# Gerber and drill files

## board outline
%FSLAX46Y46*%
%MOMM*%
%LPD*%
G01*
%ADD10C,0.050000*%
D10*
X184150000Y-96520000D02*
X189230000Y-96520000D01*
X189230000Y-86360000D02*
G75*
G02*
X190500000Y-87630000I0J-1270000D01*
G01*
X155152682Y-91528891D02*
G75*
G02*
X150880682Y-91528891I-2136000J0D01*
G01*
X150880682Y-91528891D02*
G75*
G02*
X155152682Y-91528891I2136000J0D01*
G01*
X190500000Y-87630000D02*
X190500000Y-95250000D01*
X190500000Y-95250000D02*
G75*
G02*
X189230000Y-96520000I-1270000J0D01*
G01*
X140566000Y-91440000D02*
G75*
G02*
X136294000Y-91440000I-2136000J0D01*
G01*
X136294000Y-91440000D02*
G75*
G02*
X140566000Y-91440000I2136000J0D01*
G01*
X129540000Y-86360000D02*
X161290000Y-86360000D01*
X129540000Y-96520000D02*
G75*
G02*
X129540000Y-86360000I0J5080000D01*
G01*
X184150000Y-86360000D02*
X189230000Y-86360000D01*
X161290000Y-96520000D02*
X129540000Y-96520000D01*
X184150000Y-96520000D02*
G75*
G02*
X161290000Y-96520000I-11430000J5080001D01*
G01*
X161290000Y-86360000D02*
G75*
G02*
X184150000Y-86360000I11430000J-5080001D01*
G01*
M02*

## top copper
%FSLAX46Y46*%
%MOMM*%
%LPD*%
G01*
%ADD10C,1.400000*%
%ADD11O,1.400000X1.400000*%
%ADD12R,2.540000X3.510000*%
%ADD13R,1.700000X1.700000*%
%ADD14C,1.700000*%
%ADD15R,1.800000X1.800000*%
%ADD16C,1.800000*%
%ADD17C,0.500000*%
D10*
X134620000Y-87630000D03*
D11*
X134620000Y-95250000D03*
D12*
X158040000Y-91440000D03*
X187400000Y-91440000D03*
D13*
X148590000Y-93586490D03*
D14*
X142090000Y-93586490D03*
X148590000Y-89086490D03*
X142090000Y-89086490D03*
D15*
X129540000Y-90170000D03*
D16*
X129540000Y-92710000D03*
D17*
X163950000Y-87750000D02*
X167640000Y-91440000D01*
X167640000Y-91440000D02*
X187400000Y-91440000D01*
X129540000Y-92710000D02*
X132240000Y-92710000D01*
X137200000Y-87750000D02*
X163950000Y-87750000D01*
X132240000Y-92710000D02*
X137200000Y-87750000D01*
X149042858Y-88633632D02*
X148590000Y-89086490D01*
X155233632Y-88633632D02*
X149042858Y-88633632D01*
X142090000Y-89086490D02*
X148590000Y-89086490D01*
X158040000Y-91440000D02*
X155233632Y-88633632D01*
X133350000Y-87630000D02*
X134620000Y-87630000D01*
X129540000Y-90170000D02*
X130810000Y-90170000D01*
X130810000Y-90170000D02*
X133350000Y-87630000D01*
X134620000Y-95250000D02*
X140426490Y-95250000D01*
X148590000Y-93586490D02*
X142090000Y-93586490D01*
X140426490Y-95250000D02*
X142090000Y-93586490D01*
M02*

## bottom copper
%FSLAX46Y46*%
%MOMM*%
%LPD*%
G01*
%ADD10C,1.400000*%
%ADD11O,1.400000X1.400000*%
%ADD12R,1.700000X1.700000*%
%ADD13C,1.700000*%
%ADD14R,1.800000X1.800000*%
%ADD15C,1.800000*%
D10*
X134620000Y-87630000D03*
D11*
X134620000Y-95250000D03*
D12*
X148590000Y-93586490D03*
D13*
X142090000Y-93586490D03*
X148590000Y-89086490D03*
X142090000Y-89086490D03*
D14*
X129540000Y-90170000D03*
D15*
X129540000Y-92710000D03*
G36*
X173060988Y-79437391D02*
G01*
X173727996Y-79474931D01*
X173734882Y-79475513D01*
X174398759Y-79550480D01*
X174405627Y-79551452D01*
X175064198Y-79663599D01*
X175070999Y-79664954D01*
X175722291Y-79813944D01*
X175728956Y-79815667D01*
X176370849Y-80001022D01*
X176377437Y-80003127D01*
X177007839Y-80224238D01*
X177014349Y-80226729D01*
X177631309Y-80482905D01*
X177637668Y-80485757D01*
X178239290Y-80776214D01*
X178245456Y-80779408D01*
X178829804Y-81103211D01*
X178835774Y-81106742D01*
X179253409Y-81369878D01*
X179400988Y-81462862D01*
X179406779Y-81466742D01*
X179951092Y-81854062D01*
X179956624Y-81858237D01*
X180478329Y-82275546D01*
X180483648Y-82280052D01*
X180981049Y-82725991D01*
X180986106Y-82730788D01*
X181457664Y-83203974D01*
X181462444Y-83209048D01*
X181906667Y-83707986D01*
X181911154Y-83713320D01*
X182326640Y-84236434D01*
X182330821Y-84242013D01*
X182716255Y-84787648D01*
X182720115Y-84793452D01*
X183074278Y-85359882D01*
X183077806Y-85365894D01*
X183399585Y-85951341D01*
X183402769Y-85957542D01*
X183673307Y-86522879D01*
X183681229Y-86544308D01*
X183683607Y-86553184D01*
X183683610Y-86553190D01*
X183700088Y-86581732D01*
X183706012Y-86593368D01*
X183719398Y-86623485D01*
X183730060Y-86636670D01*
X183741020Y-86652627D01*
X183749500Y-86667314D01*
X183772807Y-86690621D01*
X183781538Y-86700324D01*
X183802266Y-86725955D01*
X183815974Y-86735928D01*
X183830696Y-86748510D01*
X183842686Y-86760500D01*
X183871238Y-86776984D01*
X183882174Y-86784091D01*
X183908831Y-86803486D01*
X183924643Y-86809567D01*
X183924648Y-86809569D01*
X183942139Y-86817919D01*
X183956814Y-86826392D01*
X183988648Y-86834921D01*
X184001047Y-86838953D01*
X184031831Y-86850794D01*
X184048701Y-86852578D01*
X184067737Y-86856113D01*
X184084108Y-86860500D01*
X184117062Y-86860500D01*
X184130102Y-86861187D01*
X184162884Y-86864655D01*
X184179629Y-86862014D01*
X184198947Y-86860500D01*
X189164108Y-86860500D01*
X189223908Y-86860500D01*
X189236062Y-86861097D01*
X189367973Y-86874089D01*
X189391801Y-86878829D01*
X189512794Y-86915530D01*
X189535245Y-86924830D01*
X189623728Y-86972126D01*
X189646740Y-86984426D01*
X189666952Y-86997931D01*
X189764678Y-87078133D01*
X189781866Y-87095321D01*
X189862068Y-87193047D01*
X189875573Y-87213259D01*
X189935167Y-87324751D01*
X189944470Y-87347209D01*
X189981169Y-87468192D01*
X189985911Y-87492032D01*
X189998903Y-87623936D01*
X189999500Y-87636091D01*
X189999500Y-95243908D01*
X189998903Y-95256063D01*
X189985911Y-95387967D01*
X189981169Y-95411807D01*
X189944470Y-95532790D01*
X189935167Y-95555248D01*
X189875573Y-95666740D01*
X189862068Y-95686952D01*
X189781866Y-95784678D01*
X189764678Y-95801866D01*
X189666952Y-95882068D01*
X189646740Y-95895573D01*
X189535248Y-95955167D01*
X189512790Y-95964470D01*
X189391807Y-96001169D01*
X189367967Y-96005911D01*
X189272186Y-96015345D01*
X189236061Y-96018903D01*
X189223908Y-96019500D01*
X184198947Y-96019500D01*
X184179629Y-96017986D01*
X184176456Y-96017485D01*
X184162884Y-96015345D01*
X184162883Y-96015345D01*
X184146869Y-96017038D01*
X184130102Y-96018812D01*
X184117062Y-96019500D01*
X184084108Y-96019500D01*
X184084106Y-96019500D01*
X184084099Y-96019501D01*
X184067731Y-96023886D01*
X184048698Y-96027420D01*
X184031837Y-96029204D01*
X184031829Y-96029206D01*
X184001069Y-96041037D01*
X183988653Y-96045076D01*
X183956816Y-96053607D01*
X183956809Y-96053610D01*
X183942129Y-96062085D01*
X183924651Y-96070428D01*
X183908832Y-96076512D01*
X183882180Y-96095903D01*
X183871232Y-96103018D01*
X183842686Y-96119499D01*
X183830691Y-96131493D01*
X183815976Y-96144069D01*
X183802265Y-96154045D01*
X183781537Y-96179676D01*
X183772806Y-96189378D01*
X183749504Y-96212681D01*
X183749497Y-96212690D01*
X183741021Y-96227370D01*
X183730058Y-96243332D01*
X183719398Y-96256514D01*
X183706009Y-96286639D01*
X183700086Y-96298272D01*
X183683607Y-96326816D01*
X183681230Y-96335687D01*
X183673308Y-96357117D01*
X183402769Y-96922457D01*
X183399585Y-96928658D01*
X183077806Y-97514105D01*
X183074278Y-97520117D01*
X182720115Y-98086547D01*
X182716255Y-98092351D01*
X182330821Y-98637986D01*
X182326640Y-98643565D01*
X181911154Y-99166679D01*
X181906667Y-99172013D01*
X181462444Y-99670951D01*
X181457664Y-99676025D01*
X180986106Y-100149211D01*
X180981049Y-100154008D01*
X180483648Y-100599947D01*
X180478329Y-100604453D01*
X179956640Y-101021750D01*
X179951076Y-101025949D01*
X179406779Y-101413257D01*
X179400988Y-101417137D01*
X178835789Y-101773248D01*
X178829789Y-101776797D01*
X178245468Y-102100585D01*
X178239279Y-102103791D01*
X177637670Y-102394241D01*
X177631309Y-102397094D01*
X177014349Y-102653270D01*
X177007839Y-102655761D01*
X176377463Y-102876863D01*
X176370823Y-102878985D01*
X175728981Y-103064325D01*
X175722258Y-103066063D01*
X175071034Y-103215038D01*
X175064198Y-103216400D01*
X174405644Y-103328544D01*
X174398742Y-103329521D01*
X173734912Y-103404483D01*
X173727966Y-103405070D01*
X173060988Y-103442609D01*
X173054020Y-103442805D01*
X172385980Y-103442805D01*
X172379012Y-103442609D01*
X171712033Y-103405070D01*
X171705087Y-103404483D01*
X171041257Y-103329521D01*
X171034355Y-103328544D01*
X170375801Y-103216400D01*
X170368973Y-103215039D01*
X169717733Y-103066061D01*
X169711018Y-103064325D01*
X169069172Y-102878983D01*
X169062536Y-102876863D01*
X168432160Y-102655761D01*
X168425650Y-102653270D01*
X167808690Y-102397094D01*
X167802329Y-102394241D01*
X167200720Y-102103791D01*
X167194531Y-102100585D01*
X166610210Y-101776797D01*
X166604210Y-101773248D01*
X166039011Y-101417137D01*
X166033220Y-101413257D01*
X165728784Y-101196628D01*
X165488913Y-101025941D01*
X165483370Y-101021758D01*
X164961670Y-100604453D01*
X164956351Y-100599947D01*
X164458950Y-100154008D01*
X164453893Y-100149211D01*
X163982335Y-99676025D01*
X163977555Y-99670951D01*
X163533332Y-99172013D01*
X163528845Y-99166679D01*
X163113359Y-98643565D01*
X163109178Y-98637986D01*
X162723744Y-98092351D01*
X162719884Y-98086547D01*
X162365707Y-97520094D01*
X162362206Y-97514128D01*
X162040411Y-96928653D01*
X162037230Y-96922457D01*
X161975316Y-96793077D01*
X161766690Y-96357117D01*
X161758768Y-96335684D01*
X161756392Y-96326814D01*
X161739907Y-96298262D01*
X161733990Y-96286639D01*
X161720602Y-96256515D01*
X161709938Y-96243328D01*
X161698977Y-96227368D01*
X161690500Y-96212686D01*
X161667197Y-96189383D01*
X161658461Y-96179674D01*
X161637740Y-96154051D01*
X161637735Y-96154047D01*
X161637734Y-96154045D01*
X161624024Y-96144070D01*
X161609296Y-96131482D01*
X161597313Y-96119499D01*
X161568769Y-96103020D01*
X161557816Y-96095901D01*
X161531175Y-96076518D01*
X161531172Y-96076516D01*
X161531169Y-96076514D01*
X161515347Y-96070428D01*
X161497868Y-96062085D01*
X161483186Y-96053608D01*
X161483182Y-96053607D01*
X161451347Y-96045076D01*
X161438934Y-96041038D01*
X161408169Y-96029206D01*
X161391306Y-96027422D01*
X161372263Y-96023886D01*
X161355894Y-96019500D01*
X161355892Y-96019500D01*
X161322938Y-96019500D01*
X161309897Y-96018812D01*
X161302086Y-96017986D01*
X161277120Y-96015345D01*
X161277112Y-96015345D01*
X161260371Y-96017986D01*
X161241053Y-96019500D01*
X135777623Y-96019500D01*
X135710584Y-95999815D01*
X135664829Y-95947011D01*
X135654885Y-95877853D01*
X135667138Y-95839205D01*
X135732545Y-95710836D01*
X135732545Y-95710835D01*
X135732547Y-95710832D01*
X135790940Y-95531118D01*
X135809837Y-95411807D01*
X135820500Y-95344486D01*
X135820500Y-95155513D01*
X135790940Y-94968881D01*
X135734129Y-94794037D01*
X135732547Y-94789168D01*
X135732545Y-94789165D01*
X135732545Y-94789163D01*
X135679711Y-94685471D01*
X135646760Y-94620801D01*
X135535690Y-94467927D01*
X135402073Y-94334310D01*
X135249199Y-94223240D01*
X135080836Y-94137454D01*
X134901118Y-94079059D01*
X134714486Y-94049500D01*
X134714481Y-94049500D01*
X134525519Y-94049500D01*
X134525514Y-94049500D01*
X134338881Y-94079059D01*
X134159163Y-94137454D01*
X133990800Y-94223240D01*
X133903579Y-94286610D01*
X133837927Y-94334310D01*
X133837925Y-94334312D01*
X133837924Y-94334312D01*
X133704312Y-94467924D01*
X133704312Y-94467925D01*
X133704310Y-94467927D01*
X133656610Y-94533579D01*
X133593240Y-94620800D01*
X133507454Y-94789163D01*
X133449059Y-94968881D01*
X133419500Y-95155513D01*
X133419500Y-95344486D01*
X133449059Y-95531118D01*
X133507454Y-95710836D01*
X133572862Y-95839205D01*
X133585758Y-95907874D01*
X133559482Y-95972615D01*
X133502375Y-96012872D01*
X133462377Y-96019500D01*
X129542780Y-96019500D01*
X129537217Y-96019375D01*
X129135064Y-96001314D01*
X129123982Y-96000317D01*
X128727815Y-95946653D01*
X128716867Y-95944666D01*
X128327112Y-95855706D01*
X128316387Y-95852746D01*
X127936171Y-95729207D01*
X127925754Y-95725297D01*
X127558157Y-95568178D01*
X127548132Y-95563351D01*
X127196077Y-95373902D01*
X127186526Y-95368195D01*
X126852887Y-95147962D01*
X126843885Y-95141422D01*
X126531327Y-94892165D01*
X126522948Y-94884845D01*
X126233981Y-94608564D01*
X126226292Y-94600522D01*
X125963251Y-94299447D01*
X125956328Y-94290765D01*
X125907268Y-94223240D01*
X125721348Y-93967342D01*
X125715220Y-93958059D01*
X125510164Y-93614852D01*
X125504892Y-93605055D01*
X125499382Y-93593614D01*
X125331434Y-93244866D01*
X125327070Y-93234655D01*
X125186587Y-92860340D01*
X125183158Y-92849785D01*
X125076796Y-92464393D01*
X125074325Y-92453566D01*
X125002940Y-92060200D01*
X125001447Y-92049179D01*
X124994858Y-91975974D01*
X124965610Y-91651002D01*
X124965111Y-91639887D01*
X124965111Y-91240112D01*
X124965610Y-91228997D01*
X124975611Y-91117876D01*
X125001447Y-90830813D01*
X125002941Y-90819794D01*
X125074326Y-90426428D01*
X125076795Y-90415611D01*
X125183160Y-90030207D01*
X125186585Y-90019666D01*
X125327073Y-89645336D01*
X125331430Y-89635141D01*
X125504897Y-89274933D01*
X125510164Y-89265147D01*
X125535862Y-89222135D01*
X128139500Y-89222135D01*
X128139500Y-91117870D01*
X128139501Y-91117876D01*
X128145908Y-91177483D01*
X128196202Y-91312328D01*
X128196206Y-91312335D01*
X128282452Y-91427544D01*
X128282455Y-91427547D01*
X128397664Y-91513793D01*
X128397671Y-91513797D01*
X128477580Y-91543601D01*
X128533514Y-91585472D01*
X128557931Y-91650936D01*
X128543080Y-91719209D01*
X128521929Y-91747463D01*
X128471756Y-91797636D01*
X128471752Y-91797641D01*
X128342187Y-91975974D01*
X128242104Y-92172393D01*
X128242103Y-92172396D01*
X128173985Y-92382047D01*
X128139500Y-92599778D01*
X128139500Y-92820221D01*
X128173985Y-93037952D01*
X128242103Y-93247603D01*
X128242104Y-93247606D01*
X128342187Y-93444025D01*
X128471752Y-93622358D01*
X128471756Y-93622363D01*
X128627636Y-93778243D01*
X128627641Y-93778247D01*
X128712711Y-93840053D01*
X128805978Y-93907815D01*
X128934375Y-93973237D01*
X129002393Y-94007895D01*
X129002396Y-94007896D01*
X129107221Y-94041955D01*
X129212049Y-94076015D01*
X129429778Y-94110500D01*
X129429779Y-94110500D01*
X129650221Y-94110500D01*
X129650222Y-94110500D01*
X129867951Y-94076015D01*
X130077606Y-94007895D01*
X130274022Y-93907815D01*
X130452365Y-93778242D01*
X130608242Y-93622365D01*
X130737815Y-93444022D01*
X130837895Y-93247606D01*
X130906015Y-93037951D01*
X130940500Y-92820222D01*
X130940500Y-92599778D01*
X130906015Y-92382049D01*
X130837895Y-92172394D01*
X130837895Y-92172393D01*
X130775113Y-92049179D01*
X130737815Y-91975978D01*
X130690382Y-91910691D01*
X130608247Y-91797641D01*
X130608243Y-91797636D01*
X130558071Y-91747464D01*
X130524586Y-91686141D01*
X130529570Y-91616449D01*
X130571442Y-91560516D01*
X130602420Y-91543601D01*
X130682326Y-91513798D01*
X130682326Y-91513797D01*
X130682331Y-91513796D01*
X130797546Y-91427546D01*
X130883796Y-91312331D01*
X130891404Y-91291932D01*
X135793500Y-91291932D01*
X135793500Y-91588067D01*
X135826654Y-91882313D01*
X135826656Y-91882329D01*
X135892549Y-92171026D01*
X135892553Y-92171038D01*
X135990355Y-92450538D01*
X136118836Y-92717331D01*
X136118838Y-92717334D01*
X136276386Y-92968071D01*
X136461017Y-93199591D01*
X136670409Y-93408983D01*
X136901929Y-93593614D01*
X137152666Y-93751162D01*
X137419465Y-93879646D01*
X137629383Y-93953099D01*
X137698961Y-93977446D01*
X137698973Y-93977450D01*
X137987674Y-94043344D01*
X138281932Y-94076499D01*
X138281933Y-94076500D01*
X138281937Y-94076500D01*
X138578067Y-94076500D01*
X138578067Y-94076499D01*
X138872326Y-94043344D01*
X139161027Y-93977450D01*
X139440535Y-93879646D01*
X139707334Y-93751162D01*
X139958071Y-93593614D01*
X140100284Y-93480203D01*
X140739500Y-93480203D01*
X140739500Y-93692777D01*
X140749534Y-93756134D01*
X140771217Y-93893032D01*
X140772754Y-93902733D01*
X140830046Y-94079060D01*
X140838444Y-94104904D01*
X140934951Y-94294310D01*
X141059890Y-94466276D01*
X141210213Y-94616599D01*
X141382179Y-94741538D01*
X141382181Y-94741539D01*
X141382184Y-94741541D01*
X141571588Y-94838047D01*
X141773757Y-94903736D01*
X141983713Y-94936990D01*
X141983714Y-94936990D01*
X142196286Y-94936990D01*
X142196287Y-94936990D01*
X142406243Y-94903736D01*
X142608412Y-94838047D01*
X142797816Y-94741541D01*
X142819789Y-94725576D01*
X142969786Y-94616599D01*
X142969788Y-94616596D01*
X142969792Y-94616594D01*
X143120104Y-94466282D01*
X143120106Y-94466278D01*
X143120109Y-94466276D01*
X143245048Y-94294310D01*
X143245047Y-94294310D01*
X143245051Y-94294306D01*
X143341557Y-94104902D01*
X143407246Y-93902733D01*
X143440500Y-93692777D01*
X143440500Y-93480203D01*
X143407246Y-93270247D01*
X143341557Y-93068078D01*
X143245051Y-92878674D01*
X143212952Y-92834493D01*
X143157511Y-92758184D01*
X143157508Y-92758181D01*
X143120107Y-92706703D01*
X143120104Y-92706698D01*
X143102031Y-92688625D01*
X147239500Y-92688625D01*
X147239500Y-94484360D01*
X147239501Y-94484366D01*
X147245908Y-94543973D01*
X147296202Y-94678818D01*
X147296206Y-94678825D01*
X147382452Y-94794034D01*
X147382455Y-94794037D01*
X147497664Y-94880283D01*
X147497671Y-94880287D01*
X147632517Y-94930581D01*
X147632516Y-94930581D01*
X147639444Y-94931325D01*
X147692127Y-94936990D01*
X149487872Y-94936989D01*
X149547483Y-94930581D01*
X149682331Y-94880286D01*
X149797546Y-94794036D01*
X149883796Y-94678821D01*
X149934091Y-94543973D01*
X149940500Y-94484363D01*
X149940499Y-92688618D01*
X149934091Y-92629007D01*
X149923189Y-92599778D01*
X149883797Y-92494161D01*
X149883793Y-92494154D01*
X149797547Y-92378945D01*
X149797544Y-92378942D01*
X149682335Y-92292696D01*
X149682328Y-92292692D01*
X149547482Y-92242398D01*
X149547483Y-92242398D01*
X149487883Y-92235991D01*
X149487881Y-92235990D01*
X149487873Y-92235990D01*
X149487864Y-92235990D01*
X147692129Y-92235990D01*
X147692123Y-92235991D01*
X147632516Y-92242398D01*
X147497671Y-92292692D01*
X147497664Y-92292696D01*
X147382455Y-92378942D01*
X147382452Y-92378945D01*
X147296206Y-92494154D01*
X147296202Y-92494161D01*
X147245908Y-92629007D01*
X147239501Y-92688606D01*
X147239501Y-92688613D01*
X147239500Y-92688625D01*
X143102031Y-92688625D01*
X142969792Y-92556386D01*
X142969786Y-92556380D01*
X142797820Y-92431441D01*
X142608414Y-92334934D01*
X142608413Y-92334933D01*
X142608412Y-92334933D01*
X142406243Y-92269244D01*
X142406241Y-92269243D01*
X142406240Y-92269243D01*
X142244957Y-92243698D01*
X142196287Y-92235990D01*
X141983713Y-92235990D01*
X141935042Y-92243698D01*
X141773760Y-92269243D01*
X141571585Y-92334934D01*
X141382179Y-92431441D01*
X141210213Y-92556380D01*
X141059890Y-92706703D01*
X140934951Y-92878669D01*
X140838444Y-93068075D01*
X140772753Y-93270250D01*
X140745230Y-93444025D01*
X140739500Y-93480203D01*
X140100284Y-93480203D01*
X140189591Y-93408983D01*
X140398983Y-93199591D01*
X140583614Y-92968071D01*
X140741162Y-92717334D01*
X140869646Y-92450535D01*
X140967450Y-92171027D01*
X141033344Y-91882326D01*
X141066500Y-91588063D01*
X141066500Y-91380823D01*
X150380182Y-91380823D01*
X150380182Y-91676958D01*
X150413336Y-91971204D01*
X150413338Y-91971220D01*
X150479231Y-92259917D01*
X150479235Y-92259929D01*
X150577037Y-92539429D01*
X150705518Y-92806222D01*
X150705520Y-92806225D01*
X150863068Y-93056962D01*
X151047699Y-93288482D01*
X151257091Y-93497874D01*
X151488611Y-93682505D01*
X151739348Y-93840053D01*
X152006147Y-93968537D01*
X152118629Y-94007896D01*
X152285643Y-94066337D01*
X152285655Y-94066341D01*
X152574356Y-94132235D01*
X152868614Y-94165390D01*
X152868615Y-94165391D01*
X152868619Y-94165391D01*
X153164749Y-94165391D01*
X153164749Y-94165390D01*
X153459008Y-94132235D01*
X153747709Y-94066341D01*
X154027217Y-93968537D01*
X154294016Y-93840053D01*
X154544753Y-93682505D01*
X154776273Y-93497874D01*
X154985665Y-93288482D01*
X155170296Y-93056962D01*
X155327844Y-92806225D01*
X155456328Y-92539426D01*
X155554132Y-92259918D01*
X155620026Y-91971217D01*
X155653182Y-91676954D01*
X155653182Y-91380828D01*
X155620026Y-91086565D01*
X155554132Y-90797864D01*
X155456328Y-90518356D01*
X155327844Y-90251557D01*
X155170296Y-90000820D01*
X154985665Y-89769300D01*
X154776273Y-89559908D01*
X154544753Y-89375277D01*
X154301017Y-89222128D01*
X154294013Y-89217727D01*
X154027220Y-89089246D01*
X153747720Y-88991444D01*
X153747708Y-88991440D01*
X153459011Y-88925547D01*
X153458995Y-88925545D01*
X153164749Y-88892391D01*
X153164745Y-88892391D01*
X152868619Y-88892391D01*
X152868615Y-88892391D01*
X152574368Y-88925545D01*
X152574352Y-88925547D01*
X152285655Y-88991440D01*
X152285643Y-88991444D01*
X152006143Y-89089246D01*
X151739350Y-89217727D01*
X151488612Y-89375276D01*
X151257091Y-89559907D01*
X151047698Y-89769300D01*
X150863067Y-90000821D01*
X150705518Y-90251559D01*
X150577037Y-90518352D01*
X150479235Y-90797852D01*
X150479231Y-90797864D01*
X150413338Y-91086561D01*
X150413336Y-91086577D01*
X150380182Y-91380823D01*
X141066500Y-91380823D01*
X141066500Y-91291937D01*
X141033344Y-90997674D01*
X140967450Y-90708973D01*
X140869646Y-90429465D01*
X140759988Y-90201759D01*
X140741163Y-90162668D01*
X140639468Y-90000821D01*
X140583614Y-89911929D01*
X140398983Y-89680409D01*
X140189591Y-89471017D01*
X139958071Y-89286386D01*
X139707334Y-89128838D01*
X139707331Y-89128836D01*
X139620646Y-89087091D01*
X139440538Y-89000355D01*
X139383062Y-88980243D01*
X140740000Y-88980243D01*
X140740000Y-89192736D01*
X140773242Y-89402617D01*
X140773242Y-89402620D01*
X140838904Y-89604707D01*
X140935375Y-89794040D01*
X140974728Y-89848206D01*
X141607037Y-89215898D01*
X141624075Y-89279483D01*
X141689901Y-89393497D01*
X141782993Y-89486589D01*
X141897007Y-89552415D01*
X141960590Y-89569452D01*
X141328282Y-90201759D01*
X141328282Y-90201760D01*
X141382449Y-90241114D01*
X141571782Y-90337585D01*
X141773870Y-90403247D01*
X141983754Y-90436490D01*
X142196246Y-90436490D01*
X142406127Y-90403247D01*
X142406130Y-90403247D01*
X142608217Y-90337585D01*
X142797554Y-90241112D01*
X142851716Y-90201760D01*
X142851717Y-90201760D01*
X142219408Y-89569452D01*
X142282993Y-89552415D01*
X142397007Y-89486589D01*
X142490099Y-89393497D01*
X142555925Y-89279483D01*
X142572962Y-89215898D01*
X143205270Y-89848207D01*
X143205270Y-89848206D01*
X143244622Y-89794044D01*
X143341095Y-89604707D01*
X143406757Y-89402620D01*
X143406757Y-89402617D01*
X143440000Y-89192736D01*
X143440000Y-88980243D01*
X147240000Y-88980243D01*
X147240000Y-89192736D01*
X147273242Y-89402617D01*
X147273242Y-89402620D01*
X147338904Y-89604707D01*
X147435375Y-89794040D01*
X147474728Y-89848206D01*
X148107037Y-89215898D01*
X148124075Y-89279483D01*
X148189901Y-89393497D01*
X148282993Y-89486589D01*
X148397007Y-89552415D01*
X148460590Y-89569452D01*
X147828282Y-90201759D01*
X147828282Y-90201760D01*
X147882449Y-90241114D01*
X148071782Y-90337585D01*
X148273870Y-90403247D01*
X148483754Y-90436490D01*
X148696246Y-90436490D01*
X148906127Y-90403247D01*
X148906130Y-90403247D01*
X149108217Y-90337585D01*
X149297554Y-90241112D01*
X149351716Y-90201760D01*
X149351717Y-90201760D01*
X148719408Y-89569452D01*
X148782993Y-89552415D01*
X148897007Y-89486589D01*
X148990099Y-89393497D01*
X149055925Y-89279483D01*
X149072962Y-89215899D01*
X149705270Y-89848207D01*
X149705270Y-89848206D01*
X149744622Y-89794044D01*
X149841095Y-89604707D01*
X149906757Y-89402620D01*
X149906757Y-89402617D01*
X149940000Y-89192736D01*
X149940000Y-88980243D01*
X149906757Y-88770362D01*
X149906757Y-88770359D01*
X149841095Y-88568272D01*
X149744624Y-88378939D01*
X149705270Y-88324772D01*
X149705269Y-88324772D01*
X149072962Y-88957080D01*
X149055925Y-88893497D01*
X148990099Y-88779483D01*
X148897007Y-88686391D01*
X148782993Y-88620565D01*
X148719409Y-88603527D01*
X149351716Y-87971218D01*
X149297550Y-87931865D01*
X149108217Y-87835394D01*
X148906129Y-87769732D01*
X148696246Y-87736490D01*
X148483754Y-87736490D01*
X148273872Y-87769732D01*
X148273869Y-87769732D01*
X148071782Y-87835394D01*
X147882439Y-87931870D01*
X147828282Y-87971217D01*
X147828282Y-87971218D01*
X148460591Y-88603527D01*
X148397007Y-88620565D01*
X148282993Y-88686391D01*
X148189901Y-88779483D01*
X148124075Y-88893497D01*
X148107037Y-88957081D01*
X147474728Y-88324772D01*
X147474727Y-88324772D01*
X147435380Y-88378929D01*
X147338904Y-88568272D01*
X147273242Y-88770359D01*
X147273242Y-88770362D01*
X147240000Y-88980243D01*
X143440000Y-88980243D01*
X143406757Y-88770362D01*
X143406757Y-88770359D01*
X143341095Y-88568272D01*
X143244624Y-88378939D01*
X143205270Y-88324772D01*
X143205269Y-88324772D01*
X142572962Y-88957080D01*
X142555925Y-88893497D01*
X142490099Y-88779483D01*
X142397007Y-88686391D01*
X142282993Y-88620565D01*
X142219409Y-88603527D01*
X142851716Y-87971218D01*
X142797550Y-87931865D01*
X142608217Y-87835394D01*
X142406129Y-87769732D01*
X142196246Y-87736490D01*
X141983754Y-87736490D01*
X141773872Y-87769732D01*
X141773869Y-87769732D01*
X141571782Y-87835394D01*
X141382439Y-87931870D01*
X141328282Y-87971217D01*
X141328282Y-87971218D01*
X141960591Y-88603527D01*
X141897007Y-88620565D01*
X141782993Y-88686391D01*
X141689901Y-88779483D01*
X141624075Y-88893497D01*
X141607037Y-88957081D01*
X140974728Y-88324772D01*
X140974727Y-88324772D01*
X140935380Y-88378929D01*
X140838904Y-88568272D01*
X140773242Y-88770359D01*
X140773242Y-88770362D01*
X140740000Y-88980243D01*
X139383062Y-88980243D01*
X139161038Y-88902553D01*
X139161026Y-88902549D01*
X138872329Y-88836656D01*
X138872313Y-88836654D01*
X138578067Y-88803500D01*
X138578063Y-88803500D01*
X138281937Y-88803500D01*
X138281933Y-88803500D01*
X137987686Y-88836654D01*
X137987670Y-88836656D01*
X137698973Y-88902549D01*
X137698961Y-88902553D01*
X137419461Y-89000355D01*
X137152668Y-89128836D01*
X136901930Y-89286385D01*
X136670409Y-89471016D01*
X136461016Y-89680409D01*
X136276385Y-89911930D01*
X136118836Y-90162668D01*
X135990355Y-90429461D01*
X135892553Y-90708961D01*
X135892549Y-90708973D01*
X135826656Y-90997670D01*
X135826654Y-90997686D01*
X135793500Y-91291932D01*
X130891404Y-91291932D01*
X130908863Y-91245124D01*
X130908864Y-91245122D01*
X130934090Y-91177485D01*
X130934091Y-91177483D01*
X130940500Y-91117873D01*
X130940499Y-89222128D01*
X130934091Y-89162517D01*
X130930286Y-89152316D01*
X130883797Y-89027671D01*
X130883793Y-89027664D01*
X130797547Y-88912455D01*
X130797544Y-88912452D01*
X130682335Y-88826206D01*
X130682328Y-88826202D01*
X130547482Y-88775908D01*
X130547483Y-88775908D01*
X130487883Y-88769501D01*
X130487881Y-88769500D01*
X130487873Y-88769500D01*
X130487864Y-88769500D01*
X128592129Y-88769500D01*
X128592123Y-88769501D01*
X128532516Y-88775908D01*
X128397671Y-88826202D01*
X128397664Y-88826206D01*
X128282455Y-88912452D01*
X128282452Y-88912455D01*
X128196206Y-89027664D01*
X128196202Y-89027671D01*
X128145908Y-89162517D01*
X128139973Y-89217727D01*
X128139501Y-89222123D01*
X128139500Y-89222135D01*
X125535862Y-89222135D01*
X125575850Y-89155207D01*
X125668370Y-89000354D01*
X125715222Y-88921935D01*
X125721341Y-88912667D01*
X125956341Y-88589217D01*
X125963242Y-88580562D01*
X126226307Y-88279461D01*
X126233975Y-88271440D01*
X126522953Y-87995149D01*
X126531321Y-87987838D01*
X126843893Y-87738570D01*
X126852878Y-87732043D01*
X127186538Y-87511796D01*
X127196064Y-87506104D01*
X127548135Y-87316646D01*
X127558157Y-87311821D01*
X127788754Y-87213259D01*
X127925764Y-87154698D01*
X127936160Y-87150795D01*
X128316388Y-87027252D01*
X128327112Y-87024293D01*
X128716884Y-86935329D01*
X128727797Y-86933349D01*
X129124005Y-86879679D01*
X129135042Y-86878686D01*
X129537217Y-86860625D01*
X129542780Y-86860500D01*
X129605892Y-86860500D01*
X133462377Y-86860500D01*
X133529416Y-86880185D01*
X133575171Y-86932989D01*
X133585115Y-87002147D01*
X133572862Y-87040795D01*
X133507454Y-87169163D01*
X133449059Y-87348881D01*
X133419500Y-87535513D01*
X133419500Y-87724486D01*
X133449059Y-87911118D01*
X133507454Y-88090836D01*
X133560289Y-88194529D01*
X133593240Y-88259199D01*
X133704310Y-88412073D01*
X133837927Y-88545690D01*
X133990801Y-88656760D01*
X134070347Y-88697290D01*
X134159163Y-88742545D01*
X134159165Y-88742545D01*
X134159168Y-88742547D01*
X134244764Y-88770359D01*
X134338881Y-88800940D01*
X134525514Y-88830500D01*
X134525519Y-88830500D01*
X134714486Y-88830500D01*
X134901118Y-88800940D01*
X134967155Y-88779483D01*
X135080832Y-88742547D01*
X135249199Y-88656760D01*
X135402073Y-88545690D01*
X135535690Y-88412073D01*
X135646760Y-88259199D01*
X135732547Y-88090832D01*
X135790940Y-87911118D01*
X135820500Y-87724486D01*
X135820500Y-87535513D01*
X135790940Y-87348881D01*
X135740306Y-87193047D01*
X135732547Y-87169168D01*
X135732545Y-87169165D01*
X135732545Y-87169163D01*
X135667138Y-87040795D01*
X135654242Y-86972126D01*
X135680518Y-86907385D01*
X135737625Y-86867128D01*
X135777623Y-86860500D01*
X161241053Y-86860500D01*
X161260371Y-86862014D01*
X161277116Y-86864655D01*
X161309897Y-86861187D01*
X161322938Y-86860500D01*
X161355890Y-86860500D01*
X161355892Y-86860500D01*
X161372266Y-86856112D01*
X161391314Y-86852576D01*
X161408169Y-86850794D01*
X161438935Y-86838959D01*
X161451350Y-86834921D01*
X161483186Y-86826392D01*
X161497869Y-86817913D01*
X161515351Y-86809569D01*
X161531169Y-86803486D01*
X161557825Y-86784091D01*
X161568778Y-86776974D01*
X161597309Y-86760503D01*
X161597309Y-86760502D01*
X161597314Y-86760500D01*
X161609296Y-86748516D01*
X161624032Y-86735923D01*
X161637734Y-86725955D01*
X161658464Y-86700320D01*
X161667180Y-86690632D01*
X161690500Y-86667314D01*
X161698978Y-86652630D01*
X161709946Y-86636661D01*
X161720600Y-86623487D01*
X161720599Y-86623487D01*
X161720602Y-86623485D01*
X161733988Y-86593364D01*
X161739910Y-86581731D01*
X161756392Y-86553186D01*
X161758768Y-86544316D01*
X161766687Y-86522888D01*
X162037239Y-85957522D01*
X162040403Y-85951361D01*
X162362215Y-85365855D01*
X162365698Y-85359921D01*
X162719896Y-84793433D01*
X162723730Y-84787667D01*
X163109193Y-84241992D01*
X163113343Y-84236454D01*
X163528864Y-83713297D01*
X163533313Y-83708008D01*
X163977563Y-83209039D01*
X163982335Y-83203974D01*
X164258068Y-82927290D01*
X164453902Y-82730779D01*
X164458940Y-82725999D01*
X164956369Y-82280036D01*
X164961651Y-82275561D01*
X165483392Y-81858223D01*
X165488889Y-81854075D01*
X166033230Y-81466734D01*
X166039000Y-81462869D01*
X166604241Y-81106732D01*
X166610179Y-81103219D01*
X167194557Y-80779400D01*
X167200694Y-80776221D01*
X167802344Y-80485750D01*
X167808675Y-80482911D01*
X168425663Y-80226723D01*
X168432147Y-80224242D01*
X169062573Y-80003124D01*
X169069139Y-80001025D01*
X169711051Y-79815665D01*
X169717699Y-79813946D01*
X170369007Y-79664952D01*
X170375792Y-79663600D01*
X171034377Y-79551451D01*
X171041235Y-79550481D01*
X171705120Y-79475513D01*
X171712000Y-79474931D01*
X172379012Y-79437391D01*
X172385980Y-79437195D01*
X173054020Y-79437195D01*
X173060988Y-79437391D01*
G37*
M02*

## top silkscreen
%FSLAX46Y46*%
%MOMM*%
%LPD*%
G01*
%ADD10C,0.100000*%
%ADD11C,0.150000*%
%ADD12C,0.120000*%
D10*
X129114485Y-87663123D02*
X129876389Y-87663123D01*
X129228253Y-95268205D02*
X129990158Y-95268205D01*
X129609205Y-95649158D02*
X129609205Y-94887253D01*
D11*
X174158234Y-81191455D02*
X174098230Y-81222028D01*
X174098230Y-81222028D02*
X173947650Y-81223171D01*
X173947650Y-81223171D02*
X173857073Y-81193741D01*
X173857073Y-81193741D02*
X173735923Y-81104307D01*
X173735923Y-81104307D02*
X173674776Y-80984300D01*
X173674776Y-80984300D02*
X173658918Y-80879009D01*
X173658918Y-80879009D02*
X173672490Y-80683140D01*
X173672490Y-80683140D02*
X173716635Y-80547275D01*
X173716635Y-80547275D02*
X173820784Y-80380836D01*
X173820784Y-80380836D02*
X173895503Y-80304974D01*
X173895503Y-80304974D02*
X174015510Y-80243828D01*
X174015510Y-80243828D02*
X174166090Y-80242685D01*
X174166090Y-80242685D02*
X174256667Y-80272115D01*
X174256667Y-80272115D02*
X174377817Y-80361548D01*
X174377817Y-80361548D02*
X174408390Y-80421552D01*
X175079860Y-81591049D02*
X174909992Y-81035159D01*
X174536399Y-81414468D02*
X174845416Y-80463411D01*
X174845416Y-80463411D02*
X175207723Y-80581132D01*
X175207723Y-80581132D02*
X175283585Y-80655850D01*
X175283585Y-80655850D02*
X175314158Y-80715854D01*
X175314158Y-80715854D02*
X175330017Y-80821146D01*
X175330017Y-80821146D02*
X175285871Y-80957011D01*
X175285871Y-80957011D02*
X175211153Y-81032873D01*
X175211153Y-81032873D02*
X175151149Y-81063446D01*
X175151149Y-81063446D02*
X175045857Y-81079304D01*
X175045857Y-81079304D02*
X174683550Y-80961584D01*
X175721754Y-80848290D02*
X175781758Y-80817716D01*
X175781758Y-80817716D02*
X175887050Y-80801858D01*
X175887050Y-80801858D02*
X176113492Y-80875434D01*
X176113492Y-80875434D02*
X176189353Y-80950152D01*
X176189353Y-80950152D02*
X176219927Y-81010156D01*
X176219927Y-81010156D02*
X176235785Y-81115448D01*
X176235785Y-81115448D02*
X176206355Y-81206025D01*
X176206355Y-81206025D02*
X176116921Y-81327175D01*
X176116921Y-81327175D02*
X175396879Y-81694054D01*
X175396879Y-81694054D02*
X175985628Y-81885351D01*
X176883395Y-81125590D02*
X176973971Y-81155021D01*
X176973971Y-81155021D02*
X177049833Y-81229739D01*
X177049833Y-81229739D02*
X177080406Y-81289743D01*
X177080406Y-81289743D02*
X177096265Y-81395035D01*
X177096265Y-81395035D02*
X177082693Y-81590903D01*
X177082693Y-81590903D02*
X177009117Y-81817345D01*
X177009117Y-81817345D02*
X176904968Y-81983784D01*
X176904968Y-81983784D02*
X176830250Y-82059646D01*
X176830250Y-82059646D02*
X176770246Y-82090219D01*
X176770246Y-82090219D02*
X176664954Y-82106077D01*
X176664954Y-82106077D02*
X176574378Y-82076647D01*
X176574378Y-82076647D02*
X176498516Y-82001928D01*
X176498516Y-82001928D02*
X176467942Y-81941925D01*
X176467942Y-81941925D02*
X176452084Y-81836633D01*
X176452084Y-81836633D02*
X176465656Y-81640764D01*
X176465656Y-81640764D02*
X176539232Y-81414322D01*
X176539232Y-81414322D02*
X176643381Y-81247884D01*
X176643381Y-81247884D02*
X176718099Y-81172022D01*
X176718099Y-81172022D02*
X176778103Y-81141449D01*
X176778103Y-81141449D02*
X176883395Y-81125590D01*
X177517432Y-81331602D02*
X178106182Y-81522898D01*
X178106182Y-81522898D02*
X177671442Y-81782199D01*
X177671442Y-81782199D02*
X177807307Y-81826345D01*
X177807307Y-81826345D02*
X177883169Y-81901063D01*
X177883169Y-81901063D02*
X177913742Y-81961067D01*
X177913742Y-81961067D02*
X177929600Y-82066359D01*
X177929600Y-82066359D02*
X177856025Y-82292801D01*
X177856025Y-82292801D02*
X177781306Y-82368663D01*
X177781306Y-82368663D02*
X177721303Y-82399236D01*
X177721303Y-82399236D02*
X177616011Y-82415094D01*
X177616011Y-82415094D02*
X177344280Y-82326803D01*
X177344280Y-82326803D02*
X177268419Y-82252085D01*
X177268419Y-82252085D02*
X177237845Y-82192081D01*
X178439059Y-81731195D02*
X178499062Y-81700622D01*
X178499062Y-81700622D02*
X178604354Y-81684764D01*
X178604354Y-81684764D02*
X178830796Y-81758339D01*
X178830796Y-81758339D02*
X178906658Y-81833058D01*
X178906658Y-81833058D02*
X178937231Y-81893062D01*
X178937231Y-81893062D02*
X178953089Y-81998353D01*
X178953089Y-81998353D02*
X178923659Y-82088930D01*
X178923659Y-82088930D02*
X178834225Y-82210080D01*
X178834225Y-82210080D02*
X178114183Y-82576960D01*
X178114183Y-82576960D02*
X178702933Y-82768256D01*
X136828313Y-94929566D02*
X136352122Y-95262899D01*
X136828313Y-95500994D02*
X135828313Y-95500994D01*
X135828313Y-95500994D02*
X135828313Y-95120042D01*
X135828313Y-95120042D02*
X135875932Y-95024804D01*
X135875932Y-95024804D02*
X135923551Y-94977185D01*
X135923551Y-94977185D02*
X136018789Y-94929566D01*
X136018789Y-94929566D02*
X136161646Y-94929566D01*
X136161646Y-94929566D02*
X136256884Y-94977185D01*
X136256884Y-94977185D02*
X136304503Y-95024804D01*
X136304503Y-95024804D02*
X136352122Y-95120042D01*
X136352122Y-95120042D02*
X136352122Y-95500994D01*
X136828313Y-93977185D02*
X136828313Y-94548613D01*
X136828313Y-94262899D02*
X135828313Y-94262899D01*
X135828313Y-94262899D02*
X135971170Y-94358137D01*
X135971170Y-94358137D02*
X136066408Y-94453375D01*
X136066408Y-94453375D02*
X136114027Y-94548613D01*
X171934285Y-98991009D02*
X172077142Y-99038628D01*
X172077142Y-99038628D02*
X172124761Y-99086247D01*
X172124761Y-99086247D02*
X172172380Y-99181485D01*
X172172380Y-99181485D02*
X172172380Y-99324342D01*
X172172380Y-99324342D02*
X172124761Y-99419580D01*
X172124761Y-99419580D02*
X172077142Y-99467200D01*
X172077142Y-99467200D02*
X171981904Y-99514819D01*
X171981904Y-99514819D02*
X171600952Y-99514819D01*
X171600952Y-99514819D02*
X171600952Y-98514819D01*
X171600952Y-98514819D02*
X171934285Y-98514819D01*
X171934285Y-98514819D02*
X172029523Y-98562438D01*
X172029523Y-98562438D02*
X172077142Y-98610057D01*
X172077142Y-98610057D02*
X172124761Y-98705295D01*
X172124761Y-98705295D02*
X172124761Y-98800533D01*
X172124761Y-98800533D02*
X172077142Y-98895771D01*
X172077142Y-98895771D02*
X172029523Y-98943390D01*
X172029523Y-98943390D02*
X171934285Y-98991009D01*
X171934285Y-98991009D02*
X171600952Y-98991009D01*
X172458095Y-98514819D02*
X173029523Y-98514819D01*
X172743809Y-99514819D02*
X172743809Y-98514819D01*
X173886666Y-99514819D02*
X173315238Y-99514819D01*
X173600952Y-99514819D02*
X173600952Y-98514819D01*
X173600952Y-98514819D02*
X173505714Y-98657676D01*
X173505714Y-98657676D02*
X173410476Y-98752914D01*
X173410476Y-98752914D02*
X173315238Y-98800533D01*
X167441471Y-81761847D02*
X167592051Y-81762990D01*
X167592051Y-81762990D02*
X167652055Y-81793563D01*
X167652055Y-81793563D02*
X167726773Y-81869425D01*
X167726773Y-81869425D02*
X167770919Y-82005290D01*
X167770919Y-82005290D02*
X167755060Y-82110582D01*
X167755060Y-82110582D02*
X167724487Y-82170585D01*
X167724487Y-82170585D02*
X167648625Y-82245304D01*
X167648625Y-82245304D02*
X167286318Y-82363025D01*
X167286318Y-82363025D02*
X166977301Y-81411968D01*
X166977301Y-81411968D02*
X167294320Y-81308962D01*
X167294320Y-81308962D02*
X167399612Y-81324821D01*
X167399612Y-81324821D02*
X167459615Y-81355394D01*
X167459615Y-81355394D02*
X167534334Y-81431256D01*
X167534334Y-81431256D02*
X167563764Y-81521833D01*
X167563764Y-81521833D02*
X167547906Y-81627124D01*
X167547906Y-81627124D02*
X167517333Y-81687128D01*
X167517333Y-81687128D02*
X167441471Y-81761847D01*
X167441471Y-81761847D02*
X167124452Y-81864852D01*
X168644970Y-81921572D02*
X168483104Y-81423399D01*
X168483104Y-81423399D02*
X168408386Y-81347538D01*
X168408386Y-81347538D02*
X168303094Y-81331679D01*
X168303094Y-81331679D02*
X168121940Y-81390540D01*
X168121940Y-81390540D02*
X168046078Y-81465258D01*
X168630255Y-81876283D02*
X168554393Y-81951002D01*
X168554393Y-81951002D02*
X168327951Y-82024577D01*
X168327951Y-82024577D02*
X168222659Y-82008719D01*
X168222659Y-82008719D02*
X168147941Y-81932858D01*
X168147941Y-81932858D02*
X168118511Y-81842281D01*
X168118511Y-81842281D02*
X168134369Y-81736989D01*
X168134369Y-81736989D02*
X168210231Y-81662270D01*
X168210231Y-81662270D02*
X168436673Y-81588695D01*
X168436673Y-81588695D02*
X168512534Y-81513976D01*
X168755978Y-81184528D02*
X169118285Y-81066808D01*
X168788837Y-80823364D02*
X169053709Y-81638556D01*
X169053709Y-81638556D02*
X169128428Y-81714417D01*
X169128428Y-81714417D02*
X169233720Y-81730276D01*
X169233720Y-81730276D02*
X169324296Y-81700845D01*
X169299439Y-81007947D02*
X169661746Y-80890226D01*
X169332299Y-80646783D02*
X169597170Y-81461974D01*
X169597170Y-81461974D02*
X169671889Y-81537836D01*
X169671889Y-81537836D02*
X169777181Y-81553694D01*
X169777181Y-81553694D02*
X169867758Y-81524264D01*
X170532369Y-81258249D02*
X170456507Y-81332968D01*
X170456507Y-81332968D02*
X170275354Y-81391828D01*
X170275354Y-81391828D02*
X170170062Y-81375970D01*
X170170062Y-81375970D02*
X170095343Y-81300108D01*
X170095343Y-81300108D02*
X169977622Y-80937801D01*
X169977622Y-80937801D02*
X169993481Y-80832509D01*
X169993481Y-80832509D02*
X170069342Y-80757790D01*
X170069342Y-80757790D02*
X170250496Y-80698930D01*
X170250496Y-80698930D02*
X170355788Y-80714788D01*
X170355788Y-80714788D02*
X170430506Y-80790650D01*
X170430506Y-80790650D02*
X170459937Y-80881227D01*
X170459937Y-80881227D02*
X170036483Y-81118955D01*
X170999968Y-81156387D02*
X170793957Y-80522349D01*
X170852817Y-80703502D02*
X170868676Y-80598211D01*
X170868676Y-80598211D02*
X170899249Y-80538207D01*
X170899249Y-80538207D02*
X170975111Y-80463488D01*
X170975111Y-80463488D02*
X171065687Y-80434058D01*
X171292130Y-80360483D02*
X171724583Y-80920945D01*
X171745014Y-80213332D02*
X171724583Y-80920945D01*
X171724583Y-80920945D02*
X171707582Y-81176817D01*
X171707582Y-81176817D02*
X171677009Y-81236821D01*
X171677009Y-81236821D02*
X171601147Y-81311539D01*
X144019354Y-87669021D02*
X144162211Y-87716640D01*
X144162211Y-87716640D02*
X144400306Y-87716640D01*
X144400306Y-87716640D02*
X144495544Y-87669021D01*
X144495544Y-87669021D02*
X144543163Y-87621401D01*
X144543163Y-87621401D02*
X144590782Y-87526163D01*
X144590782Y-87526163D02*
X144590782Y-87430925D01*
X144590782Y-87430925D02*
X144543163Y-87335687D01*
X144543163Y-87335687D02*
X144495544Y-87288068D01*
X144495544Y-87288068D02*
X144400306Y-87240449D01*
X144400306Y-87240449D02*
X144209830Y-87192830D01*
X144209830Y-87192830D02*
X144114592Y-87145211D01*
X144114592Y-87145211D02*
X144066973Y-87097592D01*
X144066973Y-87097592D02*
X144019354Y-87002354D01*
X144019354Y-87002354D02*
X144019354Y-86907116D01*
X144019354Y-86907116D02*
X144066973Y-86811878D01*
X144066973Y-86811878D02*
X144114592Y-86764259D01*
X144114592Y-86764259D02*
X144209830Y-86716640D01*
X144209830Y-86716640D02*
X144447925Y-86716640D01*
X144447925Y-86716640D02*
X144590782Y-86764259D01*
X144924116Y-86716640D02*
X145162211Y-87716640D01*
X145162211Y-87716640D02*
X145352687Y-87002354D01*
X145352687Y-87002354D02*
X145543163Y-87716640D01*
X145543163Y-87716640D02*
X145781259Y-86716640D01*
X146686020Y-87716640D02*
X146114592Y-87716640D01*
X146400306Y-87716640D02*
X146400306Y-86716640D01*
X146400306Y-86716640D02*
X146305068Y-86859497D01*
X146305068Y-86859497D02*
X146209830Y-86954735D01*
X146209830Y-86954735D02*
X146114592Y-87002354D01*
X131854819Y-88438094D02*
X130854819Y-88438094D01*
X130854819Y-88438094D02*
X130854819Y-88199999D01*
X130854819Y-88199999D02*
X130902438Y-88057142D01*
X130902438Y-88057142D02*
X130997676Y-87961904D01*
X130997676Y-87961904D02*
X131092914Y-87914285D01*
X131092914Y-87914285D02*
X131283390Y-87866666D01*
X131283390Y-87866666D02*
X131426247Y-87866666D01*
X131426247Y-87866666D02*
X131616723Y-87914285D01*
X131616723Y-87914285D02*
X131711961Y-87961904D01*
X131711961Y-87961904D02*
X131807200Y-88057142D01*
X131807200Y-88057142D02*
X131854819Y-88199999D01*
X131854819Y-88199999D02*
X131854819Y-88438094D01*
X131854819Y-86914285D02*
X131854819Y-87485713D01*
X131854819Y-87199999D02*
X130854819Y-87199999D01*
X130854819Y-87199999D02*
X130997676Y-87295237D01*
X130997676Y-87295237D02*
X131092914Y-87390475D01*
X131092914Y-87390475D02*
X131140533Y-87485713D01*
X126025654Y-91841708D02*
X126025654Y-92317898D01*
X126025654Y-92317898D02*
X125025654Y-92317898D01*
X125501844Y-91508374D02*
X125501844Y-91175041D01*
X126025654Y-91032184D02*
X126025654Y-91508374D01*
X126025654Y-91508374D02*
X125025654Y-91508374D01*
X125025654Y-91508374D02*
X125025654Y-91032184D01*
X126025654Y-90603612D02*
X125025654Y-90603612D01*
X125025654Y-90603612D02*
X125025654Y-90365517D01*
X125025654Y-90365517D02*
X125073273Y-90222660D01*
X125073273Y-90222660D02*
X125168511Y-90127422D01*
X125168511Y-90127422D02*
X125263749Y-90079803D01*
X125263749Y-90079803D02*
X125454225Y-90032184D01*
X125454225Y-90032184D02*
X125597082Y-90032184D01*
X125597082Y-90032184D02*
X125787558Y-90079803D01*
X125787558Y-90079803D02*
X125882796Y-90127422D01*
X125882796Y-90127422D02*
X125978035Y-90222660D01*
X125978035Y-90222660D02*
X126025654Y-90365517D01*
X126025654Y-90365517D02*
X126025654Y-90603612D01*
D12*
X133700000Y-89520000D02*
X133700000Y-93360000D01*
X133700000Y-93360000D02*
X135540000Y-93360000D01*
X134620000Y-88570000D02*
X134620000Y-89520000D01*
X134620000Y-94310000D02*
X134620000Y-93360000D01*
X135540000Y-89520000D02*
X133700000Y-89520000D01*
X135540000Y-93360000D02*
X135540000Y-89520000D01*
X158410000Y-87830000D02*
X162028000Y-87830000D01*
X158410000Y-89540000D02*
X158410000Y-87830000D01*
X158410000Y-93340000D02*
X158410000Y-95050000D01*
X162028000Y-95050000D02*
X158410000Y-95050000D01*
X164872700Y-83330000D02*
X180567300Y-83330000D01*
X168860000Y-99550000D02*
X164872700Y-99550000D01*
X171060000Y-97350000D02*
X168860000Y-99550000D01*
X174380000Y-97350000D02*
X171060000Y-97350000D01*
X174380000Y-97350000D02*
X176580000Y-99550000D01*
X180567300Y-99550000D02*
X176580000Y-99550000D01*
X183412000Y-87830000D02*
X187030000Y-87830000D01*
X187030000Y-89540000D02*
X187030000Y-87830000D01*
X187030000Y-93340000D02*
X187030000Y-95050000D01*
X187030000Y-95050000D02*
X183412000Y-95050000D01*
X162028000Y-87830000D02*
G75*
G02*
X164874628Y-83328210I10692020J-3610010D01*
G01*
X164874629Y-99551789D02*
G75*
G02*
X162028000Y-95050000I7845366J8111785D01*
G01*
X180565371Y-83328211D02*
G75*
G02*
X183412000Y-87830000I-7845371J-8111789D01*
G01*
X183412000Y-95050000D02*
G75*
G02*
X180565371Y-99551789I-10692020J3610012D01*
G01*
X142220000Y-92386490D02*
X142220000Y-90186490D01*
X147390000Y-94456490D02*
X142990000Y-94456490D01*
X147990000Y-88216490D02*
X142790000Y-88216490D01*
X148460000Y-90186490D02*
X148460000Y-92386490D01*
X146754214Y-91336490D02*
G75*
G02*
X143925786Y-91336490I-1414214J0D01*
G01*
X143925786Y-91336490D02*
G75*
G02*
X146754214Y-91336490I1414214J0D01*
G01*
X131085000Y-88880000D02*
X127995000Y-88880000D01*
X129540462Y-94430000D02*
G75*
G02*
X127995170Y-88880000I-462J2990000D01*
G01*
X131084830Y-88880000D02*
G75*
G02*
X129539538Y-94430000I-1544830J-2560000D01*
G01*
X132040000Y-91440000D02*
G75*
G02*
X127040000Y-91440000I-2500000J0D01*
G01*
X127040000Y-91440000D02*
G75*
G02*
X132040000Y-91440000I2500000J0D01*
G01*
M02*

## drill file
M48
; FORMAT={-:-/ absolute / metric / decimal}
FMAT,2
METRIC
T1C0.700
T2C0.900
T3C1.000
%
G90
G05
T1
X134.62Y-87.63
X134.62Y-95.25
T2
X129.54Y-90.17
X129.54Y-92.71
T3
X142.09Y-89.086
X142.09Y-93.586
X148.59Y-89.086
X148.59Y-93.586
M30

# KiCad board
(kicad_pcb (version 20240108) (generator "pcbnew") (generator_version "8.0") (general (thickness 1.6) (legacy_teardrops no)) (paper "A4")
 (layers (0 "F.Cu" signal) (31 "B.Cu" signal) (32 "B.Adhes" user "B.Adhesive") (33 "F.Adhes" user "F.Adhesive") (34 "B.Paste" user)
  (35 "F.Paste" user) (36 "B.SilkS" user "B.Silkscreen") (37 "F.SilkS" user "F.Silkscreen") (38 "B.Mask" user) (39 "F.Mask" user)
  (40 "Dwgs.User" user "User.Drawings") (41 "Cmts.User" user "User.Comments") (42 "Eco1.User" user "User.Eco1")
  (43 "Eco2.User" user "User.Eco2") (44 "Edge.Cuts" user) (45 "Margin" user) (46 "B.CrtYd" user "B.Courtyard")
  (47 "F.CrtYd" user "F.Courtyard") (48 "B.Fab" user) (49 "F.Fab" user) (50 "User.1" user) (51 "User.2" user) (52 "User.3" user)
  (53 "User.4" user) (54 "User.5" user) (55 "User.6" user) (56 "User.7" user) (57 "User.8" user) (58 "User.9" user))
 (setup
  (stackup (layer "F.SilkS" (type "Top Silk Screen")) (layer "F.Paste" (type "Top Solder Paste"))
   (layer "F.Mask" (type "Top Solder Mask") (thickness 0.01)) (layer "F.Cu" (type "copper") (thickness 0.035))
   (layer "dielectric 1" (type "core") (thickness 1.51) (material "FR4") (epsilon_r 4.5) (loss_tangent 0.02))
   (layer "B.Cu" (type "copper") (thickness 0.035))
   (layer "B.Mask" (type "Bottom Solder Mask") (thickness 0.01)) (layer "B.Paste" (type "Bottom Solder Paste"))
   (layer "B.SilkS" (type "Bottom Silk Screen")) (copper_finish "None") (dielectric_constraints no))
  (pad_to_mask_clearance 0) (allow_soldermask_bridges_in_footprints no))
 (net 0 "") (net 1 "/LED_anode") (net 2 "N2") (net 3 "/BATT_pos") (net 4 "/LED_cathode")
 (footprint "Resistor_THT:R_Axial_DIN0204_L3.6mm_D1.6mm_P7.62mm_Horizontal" (layer "F.Cu") (at 134.62 87.63 -90)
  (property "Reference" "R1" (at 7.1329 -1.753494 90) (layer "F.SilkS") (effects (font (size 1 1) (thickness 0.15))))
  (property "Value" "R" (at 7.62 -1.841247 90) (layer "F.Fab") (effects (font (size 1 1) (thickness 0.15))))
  (fp_line (start 1.89 0.92) (end 5.73 0.92) (stroke (width 0.12) (type solid)) (layer "F.SilkS"))
  (fp_line (start 5.73 0.92) (end 5.73 -0.92) (stroke (width 0.12) (type solid)) (layer "F.SilkS"))
  (fp_line (start 0.94 0) (end 1.89 0) (stroke (width 0.12) (type solid)) (layer "F.SilkS"))
  (fp_line (start 6.68 0) (end 5.73 0) (stroke (width 0.12) (type solid)) (layer "F.SilkS"))
  (fp_line (start 1.89 -0.92) (end 1.89 0.92) (stroke (width 0.12) (type solid)) (layer "F.SilkS"))
  (fp_line (start 5.73 -0.92) (end 1.89 -0.92) (stroke (width 0.12) (type solid)) (layer "F.SilkS"))
  (pad "1" thru_hole circle (at 0 0 270) (size 1.4 1.4) (drill 0.7) (layers "*.Cu" "*.Mask") (remove_unused_layers no) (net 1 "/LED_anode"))
  (pad "2" thru_hole oval (at 7.62 0 270) (size 1.4 1.4) (drill 0.7) (layers "*.Cu" "*.Mask") (remove_unused_layers no) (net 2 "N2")))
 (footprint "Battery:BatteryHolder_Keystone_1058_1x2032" (layer "F.Cu") (at 172.72 91.44)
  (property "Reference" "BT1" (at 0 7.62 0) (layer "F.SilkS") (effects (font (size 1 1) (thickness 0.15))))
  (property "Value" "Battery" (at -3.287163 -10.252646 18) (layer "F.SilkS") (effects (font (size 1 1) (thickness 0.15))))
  (fp_line (start -14.31 -3.61) (end -10.692 -3.61) (stroke (width 0.12) (type solid)) (layer "F.SilkS"))
  (fp_line (start -14.31 -1.9) (end -14.31 -3.61) (stroke (width 0.12) (type solid)) (layer "F.SilkS"))
  (fp_line (start -14.31 1.9) (end -14.31 3.61) (stroke (width 0.12) (type solid)) (layer "F.SilkS"))
  (fp_line (start -10.692 3.61) (end -14.31 3.61) (stroke (width 0.12) (type solid)) (layer "F.SilkS"))
  (fp_line (start -7.8473 -8.11) (end 7.8473 -8.11) (stroke (width 0.12) (type solid)) (layer "F.SilkS"))
  (fp_line (start -3.86 8.11) (end -7.8473 8.11) (stroke (width 0.12) (type solid)) (layer "F.SilkS"))
  (fp_line (start -1.66 5.91) (end -3.86 8.11) (stroke (width 0.12) (type solid)) (layer "F.SilkS"))
  (fp_line (start 1.66 5.91) (end -1.66 5.91) (stroke (width 0.12) (type solid)) (layer "F.SilkS"))
  (fp_line (start 1.66 5.91) (end 3.86 8.11) (stroke (width 0.12) (type solid)) (layer "F.SilkS"))
  (fp_line (start 7.8473 8.11) (end 3.86 8.11) (stroke (width 0.12) (type solid)) (layer "F.SilkS"))
  (fp_line (start 10.692 -3.61) (end 14.31 -3.61) (stroke (width 0.12) (type solid)) (layer "F.SilkS"))
  (fp_line (start 14.31 -1.9) (end 14.31 -3.61) (stroke (width 0.12) (type solid)) (layer "F.SilkS"))
  (fp_line (start 14.31 1.9) (end 14.31 3.61) (stroke (width 0.12) (type solid)) (layer "F.SilkS"))
  (fp_line (start 14.31 3.61) (end 10.692 3.61) (stroke (width 0.12) (type solid)) (layer "F.SilkS"))
  (fp_arc (start -10.692 -3.61) (mid -9.538084 -6.031244) (end -7.845371 -8.111789) (stroke (width 0.12) (type solid)) (layer "F.SilkS"))
  (fp_arc (start -7.845371 8.111789) (mid -9.538085 6.031244) (end -10.692 3.61) (stroke (width 0.12) (type solid)) (layer "F.SilkS"))
  (fp_arc (start 7.845371 -8.111789) (mid 9.538085 -6.031244) (end 10.692 -3.61) (stroke (width 0.12) (type solid)) (layer "F.SilkS"))
  (fp_arc (start 10.692 3.61) (mid 9.538084 6.031244) (end 7.845371 8.111789) (stroke (width 0.12) (type solid)) (layer "F.SilkS"))
  (pad "1" smd rect (at -14.68 0) (size 2.54 3.51) (layers "F.Cu" "F.Paste" "F.Mask") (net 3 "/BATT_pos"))
  (pad "2" smd rect (at 14.68 0) (size 2.54 3.51) (layers "F.Cu" "F.Paste" "F.Mask") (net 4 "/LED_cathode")))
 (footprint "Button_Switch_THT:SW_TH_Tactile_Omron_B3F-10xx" (layer "F.Cu") (at 148.59 93.58649 180)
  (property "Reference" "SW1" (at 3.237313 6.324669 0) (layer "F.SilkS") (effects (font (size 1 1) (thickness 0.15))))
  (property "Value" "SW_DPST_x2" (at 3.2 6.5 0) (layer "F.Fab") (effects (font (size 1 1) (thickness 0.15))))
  (fp_line (start 6.37 1.2) (end 6.37 3.4) (stroke (width 0.12) (type solid)) (layer "F.SilkS"))
  (fp_line (start 1.2 -0.87) (end 5.6 -0.87) (stroke (width 0.12) (type solid)) (layer "F.SilkS"))
  (fp_line (start 0.6 5.37) (end 5.8 5.37) (stroke (width 0.12) (type solid)) (layer "F.SilkS"))
  (fp_line (start 0.13 3.4) (end 0.13 1.2) (stroke (width 0.12) (type solid)) (layer "F.SilkS"))
  (fp_circle (center 3.25 2.25) (end 4.25 3.25) (stroke (width 0.12) (type solid)) (fill none) (layer "F.SilkS"))
  (pad "1" thru_hole rect (at 0 0 180) (size 1.7 1.7) (drill 1) (layers "*.Cu" "*.Mask") (remove_unused_layers no) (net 2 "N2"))
  (pad "1" thru_hole circle (at 6.5 0 180) (size 1.7 1.7) (drill 1) (layers "*.Cu" "*.Mask") (remove_unused_layers no) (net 2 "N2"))
  (pad "2" thru_hole circle (at 0 4.5 180) (size 1.7 1.7) (drill 1) (layers "*.Cu" "*.Mask") (remove_unused_layers no) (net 3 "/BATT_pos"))
  (pad "2" thru_hole circle (at 6.5 4.5 180) (size 1.7 1.7) (drill 1) (layers "*.Cu" "*.Mask") (remove_unused_layers no) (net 3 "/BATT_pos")))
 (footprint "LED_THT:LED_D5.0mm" (layer "F.Cu") (at 129.54 90.17 -90)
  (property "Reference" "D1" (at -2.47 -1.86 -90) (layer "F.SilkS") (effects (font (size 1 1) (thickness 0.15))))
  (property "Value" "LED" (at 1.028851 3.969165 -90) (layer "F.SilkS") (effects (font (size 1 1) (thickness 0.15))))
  (fp_line (start -1.29 -1.545) (end -1.29 1.545) (stroke (width 0.12) (type solid)) (layer "F.SilkS"))
  (fp_arc (start 4.26 -0.000462) (mid 2.072002 2.880433) (end -1.29 1.54483) (stroke (width 0.12) (type solid)) (layer "F.SilkS"))
  (fp_arc (start -1.29 -1.54483) (mid 2.072002 -2.880433) (end 4.26 0.000462) (stroke (width 0.12) (type solid)) (layer "F.SilkS"))
  (fp_circle (center 1.27 0) (end 3.77 0) (stroke (width 0.12) (type solid)) (fill none) (layer "F.SilkS"))
  (pad "1" thru_hole rect (at 0 0 270) (size 1.8 1.8) (drill 0.9) (layers "*.Cu" "*.Mask") (remove_unused_layers no) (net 1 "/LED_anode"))
  (pad "2" thru_hole circle (at 2.54 0 270) (size 1.8 1.8) (drill 0.9) (layers "*.Cu" "*.Mask") (remove_unused_layers no)
   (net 4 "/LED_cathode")))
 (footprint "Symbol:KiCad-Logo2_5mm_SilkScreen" (layer "B.Cu") (at 183.392929 91.164618 180)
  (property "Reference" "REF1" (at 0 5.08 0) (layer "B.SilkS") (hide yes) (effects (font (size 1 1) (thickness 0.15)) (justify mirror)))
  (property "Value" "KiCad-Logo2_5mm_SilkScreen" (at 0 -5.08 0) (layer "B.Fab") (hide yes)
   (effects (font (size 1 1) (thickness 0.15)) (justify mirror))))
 (gr_line (start 184.15 96.52) (end 189.23 96.52) (stroke (width 0.05) (type default)) (layer "Edge.Cuts"))
 (gr_arc (start 189.23 86.36) (mid 190.128026 86.731974) (end 190.5 87.63) (stroke (width 0.05) (type default)) (layer "Edge.Cuts"))
 (gr_circle (center 153.016682 91.528891) (end 155.152682 91.528891) (stroke (width 0.05) (type default)) (fill none) (layer "Edge.Cuts"))
 (gr_line (start 190.5 87.63) (end 190.5 95.25) (stroke (width 0.05) (type default)) (layer "Edge.Cuts"))
 (gr_arc (start 190.5 95.25) (mid 190.128026 96.148026) (end 189.23 96.52) (stroke (width 0.05) (type default)) (layer "Edge.Cuts"))
 (gr_circle (center 138.43 91.44) (end 140.566 91.44) (stroke (width 0.05) (type default)) (fill none) (layer "Edge.Cuts"))
 (gr_line (start 129.54 86.36) (end 161.29 86.36) (stroke (width 0.05) (type default)) (layer "Edge.Cuts"))
 (gr_arc (start 129.54 96.52) (mid 124.46 91.44) (end 129.54 86.36) (stroke (width 0.05) (type default)) (layer "Edge.Cuts"))
 (gr_line (start 184.15 86.36) (end 189.23 86.36) (stroke (width 0.05) (type default)) (layer "Edge.Cuts"))
 (gr_line (start 161.29 96.52) (end 129.54 96.52) (stroke (width 0.05) (type default)) (layer "Edge.Cuts"))
 (gr_arc (start 184.15 96.52) (mid 172.72 103.948049) (end 161.29 96.52) (stroke (width 0.05) (type default)) (layer "Edge.Cuts"))
 (gr_arc (start 161.29 86.36) (mid 172.72 78.931951) (end 184.15 86.36) (stroke (width 0.05) (type default)) (layer "Edge.Cuts"))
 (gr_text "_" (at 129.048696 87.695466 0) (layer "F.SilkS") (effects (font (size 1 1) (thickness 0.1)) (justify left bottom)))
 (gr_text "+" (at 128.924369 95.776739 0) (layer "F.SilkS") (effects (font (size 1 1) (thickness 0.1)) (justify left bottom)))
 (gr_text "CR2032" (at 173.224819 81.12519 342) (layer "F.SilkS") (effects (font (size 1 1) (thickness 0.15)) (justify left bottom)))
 (segment (start 163.95 87.75) (end 167.64 91.44) (width 0.5) (layer "F.Cu") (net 4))
 (segment (start 167.64 91.44) (end 187.4 91.44) (width 0.5) (layer "F.Cu") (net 4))
 (segment (start 129.54 92.71) (end 132.24 92.71) (width 0.5) (layer "F.Cu") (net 4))
 (segment (start 137.2 87.75) (end 163.95 87.75) (width 0.5) (layer "F.Cu") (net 4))
 (segment (start 132.24 92.71) (end 137.2 87.75) (width 0.5) (layer "F.Cu") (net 4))
 (segment (start 149.042858 88.633632) (end 148.59 89.08649) (width 0.5) (layer "F.Cu") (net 3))
 (segment (start 155.233632 88.633632) (end 149.042858 88.633632) (width 0.5) (layer "F.Cu") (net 3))
 (segment (start 142.09 89.08649) (end 148.59 89.08649) (width 0.5) (layer "F.Cu") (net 3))
 (segment (start 158.04 91.44) (end 155.233632 88.633632) (width 0.5) (layer "F.Cu") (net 3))
 (segment (start 133.35 87.63) (end 134.62 87.63) (width 0.5) (layer "F.Cu") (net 1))
 (segment (start 129.54 90.17) (end 130.81 90.17) (width 0.5) (layer "F.Cu") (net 1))
 (segment (start 130.81 90.17) (end 133.35 87.63) (width 0.5) (layer "F.Cu") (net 1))
 (segment (start 134.62 95.25) (end 140.42649 95.25) (width 0.5) (layer "F.Cu") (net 2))
 (segment (start 148.59 93.58649) (end 142.09 93.58649) (width 0.5) (layer "F.Cu") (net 2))
 (segment (start 140.42649 95.25) (end 142.09 93.58649) (width 0.5) (layer "F.Cu") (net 2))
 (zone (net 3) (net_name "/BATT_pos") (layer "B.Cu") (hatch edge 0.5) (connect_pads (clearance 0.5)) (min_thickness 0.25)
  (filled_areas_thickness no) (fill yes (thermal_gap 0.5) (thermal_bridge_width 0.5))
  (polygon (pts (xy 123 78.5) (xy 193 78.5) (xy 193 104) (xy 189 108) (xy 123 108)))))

